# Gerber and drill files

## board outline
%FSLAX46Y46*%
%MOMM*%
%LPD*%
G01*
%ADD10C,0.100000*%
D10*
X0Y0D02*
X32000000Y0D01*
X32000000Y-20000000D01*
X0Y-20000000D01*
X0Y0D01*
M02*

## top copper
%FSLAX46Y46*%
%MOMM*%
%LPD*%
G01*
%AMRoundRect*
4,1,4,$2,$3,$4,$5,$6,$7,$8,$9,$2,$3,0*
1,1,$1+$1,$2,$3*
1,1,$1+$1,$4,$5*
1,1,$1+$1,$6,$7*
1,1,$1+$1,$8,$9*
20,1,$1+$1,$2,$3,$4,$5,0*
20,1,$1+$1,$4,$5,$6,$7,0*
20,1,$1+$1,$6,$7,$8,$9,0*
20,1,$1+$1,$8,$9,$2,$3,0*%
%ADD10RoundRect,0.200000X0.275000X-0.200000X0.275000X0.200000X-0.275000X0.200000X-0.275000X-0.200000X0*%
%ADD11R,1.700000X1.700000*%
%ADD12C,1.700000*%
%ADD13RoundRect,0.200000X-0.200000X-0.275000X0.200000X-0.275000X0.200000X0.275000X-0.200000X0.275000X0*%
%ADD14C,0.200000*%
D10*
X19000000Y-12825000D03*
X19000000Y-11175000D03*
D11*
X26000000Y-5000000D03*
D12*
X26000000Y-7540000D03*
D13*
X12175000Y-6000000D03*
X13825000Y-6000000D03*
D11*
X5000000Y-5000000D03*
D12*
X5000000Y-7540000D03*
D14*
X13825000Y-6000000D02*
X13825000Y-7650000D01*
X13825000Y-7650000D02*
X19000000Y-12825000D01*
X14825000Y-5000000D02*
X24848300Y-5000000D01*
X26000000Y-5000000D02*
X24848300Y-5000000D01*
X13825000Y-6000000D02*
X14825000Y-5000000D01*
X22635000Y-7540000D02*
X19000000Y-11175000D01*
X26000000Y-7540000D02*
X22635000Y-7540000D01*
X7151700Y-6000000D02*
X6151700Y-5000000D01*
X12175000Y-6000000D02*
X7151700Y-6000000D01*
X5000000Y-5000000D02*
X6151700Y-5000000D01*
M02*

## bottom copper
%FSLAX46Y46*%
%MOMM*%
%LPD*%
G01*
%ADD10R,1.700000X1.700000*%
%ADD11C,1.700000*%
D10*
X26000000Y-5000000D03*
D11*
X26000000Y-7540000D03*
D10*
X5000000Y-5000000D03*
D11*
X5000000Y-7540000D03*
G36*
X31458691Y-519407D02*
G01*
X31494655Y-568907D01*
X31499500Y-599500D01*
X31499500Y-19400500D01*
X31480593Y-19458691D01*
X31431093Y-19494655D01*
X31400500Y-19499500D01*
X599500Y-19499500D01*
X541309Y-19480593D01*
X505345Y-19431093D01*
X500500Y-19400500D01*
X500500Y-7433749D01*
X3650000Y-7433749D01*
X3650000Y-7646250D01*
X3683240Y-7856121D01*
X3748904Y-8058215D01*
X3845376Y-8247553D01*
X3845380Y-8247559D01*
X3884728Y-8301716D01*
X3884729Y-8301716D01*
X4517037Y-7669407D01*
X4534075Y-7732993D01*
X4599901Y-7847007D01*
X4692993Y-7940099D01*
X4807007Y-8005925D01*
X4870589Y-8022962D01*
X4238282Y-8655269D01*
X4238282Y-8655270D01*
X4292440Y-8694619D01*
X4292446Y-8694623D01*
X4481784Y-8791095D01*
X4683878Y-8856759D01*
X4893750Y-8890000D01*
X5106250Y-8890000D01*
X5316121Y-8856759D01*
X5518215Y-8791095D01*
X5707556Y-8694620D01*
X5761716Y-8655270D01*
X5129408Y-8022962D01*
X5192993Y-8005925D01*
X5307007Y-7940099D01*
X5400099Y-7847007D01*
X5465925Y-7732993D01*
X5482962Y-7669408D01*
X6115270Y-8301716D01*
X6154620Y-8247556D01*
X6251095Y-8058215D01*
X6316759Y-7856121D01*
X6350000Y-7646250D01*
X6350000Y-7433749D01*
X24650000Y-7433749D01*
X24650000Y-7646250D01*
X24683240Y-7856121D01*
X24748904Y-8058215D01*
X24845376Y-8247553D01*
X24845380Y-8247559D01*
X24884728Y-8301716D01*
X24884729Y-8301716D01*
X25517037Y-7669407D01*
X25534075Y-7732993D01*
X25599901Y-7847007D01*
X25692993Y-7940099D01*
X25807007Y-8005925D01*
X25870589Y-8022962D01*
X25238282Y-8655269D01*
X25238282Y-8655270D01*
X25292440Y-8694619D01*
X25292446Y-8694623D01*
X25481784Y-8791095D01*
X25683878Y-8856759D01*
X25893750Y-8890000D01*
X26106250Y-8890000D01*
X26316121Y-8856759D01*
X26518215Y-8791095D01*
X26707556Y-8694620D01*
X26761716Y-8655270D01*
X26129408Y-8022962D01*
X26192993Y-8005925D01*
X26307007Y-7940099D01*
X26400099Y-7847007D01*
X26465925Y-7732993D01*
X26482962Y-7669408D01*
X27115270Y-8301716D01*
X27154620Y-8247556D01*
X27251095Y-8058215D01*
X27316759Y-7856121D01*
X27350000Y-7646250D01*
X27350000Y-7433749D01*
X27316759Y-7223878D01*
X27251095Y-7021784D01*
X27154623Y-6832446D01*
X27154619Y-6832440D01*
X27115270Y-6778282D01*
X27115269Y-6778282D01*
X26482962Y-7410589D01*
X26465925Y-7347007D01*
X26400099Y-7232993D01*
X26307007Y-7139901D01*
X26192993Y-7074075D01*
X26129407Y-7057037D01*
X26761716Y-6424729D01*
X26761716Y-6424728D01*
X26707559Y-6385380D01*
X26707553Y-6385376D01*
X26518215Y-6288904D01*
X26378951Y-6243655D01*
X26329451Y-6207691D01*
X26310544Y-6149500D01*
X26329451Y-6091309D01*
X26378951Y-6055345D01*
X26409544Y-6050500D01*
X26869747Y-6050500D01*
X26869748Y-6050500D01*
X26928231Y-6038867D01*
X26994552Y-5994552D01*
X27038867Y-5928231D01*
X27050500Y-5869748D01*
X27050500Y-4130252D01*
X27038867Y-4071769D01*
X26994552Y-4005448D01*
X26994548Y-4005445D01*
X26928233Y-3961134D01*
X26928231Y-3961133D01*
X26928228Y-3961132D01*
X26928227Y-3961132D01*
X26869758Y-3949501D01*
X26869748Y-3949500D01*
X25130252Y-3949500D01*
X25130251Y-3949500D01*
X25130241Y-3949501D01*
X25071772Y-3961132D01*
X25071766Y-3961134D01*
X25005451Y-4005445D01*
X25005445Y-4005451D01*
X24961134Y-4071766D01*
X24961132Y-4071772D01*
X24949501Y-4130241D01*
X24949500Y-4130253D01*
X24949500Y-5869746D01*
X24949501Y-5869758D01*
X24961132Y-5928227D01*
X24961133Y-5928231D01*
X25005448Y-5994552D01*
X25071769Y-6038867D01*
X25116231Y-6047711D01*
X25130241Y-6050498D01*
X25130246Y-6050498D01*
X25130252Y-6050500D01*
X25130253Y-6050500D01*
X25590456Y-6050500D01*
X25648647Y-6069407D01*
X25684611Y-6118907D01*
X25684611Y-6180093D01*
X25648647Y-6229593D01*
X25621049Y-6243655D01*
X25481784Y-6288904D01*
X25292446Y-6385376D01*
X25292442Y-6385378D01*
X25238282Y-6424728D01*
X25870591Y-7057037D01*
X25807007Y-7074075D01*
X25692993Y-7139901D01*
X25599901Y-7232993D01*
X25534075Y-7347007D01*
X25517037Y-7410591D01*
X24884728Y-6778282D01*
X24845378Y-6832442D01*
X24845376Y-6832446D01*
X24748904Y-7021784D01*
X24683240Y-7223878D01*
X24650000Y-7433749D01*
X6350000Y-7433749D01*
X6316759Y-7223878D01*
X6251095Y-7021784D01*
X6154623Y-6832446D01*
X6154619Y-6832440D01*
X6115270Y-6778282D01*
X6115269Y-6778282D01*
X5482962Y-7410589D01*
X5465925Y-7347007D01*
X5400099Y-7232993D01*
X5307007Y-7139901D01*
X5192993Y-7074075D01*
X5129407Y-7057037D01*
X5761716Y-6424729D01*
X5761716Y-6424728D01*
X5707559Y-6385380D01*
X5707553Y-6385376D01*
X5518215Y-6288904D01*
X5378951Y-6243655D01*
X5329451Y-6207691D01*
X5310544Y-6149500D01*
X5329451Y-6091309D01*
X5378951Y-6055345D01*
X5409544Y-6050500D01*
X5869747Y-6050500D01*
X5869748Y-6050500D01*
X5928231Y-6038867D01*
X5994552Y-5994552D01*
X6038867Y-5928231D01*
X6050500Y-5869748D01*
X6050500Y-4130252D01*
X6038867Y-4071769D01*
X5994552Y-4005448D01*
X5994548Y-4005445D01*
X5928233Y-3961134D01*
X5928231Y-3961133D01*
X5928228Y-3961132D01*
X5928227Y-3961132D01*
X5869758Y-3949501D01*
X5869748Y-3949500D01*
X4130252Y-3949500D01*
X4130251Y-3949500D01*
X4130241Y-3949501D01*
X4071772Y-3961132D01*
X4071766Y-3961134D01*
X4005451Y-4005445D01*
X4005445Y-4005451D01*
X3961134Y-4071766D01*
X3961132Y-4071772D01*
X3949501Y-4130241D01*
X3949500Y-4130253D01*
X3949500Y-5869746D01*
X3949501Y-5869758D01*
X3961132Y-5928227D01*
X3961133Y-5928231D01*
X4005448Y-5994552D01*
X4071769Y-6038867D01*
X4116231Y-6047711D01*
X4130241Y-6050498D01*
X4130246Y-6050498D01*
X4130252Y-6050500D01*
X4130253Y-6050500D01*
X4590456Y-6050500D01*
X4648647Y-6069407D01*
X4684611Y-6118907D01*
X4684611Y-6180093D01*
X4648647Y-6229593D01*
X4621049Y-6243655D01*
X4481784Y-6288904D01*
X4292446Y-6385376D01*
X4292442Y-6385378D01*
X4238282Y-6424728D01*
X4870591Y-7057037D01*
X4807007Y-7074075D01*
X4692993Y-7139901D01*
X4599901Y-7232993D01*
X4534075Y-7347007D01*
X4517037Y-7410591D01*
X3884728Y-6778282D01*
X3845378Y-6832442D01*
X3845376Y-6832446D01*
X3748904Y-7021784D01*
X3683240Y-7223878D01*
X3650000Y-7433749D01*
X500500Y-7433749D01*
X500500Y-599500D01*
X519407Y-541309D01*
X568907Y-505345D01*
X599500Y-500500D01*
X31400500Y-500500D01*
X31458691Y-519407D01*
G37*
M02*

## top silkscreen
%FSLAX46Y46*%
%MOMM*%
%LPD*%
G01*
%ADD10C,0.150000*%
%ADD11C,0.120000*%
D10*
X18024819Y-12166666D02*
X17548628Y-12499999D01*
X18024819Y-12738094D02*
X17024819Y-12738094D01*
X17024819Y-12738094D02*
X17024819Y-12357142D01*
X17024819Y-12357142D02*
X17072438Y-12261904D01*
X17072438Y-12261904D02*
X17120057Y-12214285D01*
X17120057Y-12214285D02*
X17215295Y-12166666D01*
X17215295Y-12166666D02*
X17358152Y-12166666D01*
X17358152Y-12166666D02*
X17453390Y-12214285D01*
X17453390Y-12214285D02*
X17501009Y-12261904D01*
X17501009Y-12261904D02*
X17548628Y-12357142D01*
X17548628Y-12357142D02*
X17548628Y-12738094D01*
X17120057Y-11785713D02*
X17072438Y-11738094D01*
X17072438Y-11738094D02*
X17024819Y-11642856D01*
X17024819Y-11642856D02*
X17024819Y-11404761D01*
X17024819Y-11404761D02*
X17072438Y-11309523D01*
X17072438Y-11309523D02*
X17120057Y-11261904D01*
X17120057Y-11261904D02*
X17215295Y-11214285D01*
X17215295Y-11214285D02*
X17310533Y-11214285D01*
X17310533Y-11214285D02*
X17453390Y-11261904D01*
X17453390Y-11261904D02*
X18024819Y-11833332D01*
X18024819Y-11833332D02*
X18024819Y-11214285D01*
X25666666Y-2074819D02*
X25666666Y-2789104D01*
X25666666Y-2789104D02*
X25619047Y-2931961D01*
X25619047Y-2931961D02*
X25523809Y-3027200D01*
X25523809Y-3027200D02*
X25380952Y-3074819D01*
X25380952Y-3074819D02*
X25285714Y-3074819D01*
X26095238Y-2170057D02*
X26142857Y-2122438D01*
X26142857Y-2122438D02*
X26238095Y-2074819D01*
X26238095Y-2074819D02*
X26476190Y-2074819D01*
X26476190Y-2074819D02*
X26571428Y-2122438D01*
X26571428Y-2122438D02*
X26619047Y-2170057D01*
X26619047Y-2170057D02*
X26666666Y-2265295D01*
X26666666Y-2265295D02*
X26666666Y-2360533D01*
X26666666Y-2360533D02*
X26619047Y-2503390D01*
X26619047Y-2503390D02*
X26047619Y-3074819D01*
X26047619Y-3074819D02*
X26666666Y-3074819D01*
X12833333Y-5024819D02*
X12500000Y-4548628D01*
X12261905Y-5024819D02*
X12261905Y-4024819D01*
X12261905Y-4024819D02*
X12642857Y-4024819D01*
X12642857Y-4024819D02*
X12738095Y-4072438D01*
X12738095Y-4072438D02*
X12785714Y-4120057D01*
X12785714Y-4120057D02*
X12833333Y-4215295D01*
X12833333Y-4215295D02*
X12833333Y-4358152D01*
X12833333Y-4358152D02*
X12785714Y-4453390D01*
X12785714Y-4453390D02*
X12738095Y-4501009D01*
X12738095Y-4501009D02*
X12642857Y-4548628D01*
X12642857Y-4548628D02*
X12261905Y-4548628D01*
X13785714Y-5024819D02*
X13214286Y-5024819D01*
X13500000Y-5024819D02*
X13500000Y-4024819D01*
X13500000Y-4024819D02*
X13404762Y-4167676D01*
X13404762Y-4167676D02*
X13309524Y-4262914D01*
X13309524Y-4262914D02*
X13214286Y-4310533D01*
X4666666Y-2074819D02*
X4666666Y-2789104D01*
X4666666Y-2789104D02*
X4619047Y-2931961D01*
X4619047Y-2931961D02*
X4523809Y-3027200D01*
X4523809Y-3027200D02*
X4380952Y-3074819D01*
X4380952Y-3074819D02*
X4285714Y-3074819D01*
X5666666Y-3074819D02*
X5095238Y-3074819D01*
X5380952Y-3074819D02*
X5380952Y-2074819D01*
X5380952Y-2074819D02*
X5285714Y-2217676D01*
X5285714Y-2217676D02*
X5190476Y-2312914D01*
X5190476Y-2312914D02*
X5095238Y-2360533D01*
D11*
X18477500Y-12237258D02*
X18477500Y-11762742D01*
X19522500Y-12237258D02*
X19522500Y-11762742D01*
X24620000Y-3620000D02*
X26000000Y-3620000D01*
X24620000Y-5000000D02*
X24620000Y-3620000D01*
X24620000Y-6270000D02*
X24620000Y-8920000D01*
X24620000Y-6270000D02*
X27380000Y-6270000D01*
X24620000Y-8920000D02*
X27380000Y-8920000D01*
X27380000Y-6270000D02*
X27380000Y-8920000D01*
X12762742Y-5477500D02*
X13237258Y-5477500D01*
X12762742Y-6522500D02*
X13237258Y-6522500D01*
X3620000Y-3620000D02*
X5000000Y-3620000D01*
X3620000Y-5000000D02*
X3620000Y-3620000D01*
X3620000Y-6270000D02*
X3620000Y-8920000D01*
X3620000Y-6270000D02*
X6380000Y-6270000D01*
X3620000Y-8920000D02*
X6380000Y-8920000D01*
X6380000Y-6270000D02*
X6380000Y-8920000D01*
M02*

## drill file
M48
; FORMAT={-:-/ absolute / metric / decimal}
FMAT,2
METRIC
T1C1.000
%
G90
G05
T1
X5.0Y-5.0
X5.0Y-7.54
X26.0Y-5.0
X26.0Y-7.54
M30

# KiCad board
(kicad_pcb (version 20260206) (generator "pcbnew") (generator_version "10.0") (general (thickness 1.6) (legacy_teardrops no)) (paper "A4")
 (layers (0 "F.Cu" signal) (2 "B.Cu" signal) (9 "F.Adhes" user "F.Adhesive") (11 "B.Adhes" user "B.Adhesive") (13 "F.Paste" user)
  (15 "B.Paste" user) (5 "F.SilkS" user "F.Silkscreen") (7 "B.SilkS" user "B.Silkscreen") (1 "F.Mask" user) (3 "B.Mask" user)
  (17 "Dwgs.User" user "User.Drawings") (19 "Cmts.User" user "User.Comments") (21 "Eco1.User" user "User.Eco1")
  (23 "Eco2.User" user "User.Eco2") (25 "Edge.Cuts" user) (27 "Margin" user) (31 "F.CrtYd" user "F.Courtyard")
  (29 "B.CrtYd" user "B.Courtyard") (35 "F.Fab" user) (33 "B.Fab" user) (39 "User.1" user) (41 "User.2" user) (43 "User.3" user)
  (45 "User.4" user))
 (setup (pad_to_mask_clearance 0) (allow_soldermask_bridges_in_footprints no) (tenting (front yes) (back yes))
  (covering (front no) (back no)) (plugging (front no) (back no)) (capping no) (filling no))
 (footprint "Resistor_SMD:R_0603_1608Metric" (layer "F.Cu") (at 19 12 90)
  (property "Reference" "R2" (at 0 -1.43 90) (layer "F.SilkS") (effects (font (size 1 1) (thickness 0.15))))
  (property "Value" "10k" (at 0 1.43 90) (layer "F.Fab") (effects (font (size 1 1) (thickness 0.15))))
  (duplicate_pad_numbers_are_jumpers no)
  (fp_line (start -0.237258 -0.5225) (end 0.237258 -0.5225) (stroke (width 0.12) (type solid)) (layer "F.SilkS"))
  (fp_line (start -0.237258 0.5225) (end 0.237258 0.5225) (stroke (width 0.12) (type solid)) (layer "F.SilkS"))
  (pad "1" smd roundrect (at -0.825 0 90) (size 0.8 0.95) (layers "F.Cu" "F.Mask" "F.Paste") (roundrect_rratio 0.25) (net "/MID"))
  (pad "2" smd roundrect (at 0.825 0 90) (size 0.8 0.95) (layers "F.Cu" "F.Mask" "F.Paste") (roundrect_rratio 0.25) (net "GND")))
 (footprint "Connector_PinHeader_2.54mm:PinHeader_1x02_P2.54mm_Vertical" (layer "F.Cu") (at 26 5)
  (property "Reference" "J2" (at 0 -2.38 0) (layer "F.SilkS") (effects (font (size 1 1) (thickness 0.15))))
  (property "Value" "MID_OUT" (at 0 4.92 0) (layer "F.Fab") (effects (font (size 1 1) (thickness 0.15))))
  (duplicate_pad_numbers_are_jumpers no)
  (fp_line (start -1.38 -1.38) (end 0 -1.38) (stroke (width 0.12) (type solid)) (layer "F.SilkS"))
  (fp_line (start -1.38 0) (end -1.38 -1.38) (stroke (width 0.12) (type solid)) (layer "F.SilkS"))
  (fp_line (start -1.38 1.27) (end -1.38 3.92) (stroke (width 0.12) (type solid)) (layer "F.SilkS"))
  (fp_line (start -1.38 1.27) (end 1.38 1.27) (stroke (width 0.12) (type solid)) (layer "F.SilkS"))
  (fp_line (start -1.38 3.92) (end 1.38 3.92) (stroke (width 0.12) (type solid)) (layer "F.SilkS"))
  (fp_line (start 1.38 1.27) (end 1.38 3.92) (stroke (width 0.12) (type solid)) (layer "F.SilkS"))
  (pad "1" thru_hole rect (at 0 0) (size 1.7 1.7) (drill 1) (layers "*.Cu" "*.Mask") (remove_unused_layers no) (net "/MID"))
  (pad "2" thru_hole circle (at 0 2.54) (size 1.7 1.7) (drill 1) (layers "*.Cu" "*.Mask") (remove_unused_layers no) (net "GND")))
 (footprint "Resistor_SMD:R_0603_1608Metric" (layer "F.Cu") (at 13 6)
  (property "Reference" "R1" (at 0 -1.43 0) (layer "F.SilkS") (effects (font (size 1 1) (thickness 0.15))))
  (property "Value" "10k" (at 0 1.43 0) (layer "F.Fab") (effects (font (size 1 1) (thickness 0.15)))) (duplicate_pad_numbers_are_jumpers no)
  (fp_line (start -0.237258 -0.5225) (end 0.237258 -0.5225) (stroke (width 0.12) (type solid)) (layer "F.SilkS"))
  (fp_line (start -0.237258 0.5225) (end 0.237258 0.5225) (stroke (width 0.12) (type solid)) (layer "F.SilkS"))
  (pad "1" smd roundrect (at -0.825 0) (size 0.8 0.95) (layers "F.Cu" "F.Mask" "F.Paste") (roundrect_rratio 0.25) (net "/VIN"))
  (pad "2" smd roundrect (at 0.825 0) (size 0.8 0.95) (layers "F.Cu" "F.Mask" "F.Paste") (roundrect_rratio 0.25) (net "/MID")))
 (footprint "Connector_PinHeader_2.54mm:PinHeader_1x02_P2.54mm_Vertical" (layer "F.Cu") (at 5 5)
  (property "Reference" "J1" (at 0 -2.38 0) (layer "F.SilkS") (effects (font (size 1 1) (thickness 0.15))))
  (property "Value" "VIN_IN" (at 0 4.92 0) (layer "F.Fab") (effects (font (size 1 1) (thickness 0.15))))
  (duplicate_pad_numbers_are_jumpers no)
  (fp_line (start -1.38 -1.38) (end 0 -1.38) (stroke (width 0.12) (type solid)) (layer "F.SilkS"))
  (fp_line (start -1.38 0) (end -1.38 -1.38) (stroke (width 0.12) (type solid)) (layer "F.SilkS"))
  (fp_line (start -1.38 1.27) (end -1.38 3.92) (stroke (width 0.12) (type solid)) (layer "F.SilkS"))
  (fp_line (start -1.38 1.27) (end 1.38 1.27) (stroke (width 0.12) (type solid)) (layer "F.SilkS"))
  (fp_line (start -1.38 3.92) (end 1.38 3.92) (stroke (width 0.12) (type solid)) (layer "F.SilkS"))
  (fp_line (start 1.38 1.27) (end 1.38 3.92) (stroke (width 0.12) (type solid)) (layer "F.SilkS"))
  (pad "1" thru_hole rect (at 0 0) (size 1.7 1.7) (drill 1) (layers "*.Cu" "*.Mask") (remove_unused_layers no) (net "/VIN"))
  (pad "2" thru_hole circle (at 0 2.54) (size 1.7 1.7) (drill 1) (layers "*.Cu" "*.Mask") (remove_unused_layers no) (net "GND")))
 (gr_rect (start 0 0) (end 32 20) (stroke (width 0.1) (type default)) (fill no) (layer "Edge.Cuts"))
 (segment (start 13.825 6) (end 13.825 7.65) (width 0.2) (layer "F.Cu") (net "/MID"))
 (segment (start 13.825 7.65) (end 19 12.825) (width 0.2) (layer "F.Cu") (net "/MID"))
 (segment (start 14.825 5) (end 24.8483 5) (width 0.2) (layer "F.Cu") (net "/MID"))
 (segment (start 26 5) (end 24.8483 5) (width 0.2) (layer "F.Cu") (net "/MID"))
 (segment (start 13.825 6) (end 14.825 5) (width 0.2) (layer "F.Cu") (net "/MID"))
 (segment (start 22.635 7.54) (end 19 11.175) (width 0.2) (layer "F.Cu") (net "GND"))
 (segment (start 26 7.54) (end 22.635 7.54) (width 0.2) (layer "F.Cu") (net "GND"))
 (segment (start 7.1517 6) (end 6.1517 5) (width 0.2) (layer "F.Cu") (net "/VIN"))
 (segment (start 12.175 6) (end 7.1517 6) (width 0.2) (layer "F.Cu") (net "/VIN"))
 (segment (start 5 5) (end 6.1517 5) (width 0.2) (layer "F.Cu") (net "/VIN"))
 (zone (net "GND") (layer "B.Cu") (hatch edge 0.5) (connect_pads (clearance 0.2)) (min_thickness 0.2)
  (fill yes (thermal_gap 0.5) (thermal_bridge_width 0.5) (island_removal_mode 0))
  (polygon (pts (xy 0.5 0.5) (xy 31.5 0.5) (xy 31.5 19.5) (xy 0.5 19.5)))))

